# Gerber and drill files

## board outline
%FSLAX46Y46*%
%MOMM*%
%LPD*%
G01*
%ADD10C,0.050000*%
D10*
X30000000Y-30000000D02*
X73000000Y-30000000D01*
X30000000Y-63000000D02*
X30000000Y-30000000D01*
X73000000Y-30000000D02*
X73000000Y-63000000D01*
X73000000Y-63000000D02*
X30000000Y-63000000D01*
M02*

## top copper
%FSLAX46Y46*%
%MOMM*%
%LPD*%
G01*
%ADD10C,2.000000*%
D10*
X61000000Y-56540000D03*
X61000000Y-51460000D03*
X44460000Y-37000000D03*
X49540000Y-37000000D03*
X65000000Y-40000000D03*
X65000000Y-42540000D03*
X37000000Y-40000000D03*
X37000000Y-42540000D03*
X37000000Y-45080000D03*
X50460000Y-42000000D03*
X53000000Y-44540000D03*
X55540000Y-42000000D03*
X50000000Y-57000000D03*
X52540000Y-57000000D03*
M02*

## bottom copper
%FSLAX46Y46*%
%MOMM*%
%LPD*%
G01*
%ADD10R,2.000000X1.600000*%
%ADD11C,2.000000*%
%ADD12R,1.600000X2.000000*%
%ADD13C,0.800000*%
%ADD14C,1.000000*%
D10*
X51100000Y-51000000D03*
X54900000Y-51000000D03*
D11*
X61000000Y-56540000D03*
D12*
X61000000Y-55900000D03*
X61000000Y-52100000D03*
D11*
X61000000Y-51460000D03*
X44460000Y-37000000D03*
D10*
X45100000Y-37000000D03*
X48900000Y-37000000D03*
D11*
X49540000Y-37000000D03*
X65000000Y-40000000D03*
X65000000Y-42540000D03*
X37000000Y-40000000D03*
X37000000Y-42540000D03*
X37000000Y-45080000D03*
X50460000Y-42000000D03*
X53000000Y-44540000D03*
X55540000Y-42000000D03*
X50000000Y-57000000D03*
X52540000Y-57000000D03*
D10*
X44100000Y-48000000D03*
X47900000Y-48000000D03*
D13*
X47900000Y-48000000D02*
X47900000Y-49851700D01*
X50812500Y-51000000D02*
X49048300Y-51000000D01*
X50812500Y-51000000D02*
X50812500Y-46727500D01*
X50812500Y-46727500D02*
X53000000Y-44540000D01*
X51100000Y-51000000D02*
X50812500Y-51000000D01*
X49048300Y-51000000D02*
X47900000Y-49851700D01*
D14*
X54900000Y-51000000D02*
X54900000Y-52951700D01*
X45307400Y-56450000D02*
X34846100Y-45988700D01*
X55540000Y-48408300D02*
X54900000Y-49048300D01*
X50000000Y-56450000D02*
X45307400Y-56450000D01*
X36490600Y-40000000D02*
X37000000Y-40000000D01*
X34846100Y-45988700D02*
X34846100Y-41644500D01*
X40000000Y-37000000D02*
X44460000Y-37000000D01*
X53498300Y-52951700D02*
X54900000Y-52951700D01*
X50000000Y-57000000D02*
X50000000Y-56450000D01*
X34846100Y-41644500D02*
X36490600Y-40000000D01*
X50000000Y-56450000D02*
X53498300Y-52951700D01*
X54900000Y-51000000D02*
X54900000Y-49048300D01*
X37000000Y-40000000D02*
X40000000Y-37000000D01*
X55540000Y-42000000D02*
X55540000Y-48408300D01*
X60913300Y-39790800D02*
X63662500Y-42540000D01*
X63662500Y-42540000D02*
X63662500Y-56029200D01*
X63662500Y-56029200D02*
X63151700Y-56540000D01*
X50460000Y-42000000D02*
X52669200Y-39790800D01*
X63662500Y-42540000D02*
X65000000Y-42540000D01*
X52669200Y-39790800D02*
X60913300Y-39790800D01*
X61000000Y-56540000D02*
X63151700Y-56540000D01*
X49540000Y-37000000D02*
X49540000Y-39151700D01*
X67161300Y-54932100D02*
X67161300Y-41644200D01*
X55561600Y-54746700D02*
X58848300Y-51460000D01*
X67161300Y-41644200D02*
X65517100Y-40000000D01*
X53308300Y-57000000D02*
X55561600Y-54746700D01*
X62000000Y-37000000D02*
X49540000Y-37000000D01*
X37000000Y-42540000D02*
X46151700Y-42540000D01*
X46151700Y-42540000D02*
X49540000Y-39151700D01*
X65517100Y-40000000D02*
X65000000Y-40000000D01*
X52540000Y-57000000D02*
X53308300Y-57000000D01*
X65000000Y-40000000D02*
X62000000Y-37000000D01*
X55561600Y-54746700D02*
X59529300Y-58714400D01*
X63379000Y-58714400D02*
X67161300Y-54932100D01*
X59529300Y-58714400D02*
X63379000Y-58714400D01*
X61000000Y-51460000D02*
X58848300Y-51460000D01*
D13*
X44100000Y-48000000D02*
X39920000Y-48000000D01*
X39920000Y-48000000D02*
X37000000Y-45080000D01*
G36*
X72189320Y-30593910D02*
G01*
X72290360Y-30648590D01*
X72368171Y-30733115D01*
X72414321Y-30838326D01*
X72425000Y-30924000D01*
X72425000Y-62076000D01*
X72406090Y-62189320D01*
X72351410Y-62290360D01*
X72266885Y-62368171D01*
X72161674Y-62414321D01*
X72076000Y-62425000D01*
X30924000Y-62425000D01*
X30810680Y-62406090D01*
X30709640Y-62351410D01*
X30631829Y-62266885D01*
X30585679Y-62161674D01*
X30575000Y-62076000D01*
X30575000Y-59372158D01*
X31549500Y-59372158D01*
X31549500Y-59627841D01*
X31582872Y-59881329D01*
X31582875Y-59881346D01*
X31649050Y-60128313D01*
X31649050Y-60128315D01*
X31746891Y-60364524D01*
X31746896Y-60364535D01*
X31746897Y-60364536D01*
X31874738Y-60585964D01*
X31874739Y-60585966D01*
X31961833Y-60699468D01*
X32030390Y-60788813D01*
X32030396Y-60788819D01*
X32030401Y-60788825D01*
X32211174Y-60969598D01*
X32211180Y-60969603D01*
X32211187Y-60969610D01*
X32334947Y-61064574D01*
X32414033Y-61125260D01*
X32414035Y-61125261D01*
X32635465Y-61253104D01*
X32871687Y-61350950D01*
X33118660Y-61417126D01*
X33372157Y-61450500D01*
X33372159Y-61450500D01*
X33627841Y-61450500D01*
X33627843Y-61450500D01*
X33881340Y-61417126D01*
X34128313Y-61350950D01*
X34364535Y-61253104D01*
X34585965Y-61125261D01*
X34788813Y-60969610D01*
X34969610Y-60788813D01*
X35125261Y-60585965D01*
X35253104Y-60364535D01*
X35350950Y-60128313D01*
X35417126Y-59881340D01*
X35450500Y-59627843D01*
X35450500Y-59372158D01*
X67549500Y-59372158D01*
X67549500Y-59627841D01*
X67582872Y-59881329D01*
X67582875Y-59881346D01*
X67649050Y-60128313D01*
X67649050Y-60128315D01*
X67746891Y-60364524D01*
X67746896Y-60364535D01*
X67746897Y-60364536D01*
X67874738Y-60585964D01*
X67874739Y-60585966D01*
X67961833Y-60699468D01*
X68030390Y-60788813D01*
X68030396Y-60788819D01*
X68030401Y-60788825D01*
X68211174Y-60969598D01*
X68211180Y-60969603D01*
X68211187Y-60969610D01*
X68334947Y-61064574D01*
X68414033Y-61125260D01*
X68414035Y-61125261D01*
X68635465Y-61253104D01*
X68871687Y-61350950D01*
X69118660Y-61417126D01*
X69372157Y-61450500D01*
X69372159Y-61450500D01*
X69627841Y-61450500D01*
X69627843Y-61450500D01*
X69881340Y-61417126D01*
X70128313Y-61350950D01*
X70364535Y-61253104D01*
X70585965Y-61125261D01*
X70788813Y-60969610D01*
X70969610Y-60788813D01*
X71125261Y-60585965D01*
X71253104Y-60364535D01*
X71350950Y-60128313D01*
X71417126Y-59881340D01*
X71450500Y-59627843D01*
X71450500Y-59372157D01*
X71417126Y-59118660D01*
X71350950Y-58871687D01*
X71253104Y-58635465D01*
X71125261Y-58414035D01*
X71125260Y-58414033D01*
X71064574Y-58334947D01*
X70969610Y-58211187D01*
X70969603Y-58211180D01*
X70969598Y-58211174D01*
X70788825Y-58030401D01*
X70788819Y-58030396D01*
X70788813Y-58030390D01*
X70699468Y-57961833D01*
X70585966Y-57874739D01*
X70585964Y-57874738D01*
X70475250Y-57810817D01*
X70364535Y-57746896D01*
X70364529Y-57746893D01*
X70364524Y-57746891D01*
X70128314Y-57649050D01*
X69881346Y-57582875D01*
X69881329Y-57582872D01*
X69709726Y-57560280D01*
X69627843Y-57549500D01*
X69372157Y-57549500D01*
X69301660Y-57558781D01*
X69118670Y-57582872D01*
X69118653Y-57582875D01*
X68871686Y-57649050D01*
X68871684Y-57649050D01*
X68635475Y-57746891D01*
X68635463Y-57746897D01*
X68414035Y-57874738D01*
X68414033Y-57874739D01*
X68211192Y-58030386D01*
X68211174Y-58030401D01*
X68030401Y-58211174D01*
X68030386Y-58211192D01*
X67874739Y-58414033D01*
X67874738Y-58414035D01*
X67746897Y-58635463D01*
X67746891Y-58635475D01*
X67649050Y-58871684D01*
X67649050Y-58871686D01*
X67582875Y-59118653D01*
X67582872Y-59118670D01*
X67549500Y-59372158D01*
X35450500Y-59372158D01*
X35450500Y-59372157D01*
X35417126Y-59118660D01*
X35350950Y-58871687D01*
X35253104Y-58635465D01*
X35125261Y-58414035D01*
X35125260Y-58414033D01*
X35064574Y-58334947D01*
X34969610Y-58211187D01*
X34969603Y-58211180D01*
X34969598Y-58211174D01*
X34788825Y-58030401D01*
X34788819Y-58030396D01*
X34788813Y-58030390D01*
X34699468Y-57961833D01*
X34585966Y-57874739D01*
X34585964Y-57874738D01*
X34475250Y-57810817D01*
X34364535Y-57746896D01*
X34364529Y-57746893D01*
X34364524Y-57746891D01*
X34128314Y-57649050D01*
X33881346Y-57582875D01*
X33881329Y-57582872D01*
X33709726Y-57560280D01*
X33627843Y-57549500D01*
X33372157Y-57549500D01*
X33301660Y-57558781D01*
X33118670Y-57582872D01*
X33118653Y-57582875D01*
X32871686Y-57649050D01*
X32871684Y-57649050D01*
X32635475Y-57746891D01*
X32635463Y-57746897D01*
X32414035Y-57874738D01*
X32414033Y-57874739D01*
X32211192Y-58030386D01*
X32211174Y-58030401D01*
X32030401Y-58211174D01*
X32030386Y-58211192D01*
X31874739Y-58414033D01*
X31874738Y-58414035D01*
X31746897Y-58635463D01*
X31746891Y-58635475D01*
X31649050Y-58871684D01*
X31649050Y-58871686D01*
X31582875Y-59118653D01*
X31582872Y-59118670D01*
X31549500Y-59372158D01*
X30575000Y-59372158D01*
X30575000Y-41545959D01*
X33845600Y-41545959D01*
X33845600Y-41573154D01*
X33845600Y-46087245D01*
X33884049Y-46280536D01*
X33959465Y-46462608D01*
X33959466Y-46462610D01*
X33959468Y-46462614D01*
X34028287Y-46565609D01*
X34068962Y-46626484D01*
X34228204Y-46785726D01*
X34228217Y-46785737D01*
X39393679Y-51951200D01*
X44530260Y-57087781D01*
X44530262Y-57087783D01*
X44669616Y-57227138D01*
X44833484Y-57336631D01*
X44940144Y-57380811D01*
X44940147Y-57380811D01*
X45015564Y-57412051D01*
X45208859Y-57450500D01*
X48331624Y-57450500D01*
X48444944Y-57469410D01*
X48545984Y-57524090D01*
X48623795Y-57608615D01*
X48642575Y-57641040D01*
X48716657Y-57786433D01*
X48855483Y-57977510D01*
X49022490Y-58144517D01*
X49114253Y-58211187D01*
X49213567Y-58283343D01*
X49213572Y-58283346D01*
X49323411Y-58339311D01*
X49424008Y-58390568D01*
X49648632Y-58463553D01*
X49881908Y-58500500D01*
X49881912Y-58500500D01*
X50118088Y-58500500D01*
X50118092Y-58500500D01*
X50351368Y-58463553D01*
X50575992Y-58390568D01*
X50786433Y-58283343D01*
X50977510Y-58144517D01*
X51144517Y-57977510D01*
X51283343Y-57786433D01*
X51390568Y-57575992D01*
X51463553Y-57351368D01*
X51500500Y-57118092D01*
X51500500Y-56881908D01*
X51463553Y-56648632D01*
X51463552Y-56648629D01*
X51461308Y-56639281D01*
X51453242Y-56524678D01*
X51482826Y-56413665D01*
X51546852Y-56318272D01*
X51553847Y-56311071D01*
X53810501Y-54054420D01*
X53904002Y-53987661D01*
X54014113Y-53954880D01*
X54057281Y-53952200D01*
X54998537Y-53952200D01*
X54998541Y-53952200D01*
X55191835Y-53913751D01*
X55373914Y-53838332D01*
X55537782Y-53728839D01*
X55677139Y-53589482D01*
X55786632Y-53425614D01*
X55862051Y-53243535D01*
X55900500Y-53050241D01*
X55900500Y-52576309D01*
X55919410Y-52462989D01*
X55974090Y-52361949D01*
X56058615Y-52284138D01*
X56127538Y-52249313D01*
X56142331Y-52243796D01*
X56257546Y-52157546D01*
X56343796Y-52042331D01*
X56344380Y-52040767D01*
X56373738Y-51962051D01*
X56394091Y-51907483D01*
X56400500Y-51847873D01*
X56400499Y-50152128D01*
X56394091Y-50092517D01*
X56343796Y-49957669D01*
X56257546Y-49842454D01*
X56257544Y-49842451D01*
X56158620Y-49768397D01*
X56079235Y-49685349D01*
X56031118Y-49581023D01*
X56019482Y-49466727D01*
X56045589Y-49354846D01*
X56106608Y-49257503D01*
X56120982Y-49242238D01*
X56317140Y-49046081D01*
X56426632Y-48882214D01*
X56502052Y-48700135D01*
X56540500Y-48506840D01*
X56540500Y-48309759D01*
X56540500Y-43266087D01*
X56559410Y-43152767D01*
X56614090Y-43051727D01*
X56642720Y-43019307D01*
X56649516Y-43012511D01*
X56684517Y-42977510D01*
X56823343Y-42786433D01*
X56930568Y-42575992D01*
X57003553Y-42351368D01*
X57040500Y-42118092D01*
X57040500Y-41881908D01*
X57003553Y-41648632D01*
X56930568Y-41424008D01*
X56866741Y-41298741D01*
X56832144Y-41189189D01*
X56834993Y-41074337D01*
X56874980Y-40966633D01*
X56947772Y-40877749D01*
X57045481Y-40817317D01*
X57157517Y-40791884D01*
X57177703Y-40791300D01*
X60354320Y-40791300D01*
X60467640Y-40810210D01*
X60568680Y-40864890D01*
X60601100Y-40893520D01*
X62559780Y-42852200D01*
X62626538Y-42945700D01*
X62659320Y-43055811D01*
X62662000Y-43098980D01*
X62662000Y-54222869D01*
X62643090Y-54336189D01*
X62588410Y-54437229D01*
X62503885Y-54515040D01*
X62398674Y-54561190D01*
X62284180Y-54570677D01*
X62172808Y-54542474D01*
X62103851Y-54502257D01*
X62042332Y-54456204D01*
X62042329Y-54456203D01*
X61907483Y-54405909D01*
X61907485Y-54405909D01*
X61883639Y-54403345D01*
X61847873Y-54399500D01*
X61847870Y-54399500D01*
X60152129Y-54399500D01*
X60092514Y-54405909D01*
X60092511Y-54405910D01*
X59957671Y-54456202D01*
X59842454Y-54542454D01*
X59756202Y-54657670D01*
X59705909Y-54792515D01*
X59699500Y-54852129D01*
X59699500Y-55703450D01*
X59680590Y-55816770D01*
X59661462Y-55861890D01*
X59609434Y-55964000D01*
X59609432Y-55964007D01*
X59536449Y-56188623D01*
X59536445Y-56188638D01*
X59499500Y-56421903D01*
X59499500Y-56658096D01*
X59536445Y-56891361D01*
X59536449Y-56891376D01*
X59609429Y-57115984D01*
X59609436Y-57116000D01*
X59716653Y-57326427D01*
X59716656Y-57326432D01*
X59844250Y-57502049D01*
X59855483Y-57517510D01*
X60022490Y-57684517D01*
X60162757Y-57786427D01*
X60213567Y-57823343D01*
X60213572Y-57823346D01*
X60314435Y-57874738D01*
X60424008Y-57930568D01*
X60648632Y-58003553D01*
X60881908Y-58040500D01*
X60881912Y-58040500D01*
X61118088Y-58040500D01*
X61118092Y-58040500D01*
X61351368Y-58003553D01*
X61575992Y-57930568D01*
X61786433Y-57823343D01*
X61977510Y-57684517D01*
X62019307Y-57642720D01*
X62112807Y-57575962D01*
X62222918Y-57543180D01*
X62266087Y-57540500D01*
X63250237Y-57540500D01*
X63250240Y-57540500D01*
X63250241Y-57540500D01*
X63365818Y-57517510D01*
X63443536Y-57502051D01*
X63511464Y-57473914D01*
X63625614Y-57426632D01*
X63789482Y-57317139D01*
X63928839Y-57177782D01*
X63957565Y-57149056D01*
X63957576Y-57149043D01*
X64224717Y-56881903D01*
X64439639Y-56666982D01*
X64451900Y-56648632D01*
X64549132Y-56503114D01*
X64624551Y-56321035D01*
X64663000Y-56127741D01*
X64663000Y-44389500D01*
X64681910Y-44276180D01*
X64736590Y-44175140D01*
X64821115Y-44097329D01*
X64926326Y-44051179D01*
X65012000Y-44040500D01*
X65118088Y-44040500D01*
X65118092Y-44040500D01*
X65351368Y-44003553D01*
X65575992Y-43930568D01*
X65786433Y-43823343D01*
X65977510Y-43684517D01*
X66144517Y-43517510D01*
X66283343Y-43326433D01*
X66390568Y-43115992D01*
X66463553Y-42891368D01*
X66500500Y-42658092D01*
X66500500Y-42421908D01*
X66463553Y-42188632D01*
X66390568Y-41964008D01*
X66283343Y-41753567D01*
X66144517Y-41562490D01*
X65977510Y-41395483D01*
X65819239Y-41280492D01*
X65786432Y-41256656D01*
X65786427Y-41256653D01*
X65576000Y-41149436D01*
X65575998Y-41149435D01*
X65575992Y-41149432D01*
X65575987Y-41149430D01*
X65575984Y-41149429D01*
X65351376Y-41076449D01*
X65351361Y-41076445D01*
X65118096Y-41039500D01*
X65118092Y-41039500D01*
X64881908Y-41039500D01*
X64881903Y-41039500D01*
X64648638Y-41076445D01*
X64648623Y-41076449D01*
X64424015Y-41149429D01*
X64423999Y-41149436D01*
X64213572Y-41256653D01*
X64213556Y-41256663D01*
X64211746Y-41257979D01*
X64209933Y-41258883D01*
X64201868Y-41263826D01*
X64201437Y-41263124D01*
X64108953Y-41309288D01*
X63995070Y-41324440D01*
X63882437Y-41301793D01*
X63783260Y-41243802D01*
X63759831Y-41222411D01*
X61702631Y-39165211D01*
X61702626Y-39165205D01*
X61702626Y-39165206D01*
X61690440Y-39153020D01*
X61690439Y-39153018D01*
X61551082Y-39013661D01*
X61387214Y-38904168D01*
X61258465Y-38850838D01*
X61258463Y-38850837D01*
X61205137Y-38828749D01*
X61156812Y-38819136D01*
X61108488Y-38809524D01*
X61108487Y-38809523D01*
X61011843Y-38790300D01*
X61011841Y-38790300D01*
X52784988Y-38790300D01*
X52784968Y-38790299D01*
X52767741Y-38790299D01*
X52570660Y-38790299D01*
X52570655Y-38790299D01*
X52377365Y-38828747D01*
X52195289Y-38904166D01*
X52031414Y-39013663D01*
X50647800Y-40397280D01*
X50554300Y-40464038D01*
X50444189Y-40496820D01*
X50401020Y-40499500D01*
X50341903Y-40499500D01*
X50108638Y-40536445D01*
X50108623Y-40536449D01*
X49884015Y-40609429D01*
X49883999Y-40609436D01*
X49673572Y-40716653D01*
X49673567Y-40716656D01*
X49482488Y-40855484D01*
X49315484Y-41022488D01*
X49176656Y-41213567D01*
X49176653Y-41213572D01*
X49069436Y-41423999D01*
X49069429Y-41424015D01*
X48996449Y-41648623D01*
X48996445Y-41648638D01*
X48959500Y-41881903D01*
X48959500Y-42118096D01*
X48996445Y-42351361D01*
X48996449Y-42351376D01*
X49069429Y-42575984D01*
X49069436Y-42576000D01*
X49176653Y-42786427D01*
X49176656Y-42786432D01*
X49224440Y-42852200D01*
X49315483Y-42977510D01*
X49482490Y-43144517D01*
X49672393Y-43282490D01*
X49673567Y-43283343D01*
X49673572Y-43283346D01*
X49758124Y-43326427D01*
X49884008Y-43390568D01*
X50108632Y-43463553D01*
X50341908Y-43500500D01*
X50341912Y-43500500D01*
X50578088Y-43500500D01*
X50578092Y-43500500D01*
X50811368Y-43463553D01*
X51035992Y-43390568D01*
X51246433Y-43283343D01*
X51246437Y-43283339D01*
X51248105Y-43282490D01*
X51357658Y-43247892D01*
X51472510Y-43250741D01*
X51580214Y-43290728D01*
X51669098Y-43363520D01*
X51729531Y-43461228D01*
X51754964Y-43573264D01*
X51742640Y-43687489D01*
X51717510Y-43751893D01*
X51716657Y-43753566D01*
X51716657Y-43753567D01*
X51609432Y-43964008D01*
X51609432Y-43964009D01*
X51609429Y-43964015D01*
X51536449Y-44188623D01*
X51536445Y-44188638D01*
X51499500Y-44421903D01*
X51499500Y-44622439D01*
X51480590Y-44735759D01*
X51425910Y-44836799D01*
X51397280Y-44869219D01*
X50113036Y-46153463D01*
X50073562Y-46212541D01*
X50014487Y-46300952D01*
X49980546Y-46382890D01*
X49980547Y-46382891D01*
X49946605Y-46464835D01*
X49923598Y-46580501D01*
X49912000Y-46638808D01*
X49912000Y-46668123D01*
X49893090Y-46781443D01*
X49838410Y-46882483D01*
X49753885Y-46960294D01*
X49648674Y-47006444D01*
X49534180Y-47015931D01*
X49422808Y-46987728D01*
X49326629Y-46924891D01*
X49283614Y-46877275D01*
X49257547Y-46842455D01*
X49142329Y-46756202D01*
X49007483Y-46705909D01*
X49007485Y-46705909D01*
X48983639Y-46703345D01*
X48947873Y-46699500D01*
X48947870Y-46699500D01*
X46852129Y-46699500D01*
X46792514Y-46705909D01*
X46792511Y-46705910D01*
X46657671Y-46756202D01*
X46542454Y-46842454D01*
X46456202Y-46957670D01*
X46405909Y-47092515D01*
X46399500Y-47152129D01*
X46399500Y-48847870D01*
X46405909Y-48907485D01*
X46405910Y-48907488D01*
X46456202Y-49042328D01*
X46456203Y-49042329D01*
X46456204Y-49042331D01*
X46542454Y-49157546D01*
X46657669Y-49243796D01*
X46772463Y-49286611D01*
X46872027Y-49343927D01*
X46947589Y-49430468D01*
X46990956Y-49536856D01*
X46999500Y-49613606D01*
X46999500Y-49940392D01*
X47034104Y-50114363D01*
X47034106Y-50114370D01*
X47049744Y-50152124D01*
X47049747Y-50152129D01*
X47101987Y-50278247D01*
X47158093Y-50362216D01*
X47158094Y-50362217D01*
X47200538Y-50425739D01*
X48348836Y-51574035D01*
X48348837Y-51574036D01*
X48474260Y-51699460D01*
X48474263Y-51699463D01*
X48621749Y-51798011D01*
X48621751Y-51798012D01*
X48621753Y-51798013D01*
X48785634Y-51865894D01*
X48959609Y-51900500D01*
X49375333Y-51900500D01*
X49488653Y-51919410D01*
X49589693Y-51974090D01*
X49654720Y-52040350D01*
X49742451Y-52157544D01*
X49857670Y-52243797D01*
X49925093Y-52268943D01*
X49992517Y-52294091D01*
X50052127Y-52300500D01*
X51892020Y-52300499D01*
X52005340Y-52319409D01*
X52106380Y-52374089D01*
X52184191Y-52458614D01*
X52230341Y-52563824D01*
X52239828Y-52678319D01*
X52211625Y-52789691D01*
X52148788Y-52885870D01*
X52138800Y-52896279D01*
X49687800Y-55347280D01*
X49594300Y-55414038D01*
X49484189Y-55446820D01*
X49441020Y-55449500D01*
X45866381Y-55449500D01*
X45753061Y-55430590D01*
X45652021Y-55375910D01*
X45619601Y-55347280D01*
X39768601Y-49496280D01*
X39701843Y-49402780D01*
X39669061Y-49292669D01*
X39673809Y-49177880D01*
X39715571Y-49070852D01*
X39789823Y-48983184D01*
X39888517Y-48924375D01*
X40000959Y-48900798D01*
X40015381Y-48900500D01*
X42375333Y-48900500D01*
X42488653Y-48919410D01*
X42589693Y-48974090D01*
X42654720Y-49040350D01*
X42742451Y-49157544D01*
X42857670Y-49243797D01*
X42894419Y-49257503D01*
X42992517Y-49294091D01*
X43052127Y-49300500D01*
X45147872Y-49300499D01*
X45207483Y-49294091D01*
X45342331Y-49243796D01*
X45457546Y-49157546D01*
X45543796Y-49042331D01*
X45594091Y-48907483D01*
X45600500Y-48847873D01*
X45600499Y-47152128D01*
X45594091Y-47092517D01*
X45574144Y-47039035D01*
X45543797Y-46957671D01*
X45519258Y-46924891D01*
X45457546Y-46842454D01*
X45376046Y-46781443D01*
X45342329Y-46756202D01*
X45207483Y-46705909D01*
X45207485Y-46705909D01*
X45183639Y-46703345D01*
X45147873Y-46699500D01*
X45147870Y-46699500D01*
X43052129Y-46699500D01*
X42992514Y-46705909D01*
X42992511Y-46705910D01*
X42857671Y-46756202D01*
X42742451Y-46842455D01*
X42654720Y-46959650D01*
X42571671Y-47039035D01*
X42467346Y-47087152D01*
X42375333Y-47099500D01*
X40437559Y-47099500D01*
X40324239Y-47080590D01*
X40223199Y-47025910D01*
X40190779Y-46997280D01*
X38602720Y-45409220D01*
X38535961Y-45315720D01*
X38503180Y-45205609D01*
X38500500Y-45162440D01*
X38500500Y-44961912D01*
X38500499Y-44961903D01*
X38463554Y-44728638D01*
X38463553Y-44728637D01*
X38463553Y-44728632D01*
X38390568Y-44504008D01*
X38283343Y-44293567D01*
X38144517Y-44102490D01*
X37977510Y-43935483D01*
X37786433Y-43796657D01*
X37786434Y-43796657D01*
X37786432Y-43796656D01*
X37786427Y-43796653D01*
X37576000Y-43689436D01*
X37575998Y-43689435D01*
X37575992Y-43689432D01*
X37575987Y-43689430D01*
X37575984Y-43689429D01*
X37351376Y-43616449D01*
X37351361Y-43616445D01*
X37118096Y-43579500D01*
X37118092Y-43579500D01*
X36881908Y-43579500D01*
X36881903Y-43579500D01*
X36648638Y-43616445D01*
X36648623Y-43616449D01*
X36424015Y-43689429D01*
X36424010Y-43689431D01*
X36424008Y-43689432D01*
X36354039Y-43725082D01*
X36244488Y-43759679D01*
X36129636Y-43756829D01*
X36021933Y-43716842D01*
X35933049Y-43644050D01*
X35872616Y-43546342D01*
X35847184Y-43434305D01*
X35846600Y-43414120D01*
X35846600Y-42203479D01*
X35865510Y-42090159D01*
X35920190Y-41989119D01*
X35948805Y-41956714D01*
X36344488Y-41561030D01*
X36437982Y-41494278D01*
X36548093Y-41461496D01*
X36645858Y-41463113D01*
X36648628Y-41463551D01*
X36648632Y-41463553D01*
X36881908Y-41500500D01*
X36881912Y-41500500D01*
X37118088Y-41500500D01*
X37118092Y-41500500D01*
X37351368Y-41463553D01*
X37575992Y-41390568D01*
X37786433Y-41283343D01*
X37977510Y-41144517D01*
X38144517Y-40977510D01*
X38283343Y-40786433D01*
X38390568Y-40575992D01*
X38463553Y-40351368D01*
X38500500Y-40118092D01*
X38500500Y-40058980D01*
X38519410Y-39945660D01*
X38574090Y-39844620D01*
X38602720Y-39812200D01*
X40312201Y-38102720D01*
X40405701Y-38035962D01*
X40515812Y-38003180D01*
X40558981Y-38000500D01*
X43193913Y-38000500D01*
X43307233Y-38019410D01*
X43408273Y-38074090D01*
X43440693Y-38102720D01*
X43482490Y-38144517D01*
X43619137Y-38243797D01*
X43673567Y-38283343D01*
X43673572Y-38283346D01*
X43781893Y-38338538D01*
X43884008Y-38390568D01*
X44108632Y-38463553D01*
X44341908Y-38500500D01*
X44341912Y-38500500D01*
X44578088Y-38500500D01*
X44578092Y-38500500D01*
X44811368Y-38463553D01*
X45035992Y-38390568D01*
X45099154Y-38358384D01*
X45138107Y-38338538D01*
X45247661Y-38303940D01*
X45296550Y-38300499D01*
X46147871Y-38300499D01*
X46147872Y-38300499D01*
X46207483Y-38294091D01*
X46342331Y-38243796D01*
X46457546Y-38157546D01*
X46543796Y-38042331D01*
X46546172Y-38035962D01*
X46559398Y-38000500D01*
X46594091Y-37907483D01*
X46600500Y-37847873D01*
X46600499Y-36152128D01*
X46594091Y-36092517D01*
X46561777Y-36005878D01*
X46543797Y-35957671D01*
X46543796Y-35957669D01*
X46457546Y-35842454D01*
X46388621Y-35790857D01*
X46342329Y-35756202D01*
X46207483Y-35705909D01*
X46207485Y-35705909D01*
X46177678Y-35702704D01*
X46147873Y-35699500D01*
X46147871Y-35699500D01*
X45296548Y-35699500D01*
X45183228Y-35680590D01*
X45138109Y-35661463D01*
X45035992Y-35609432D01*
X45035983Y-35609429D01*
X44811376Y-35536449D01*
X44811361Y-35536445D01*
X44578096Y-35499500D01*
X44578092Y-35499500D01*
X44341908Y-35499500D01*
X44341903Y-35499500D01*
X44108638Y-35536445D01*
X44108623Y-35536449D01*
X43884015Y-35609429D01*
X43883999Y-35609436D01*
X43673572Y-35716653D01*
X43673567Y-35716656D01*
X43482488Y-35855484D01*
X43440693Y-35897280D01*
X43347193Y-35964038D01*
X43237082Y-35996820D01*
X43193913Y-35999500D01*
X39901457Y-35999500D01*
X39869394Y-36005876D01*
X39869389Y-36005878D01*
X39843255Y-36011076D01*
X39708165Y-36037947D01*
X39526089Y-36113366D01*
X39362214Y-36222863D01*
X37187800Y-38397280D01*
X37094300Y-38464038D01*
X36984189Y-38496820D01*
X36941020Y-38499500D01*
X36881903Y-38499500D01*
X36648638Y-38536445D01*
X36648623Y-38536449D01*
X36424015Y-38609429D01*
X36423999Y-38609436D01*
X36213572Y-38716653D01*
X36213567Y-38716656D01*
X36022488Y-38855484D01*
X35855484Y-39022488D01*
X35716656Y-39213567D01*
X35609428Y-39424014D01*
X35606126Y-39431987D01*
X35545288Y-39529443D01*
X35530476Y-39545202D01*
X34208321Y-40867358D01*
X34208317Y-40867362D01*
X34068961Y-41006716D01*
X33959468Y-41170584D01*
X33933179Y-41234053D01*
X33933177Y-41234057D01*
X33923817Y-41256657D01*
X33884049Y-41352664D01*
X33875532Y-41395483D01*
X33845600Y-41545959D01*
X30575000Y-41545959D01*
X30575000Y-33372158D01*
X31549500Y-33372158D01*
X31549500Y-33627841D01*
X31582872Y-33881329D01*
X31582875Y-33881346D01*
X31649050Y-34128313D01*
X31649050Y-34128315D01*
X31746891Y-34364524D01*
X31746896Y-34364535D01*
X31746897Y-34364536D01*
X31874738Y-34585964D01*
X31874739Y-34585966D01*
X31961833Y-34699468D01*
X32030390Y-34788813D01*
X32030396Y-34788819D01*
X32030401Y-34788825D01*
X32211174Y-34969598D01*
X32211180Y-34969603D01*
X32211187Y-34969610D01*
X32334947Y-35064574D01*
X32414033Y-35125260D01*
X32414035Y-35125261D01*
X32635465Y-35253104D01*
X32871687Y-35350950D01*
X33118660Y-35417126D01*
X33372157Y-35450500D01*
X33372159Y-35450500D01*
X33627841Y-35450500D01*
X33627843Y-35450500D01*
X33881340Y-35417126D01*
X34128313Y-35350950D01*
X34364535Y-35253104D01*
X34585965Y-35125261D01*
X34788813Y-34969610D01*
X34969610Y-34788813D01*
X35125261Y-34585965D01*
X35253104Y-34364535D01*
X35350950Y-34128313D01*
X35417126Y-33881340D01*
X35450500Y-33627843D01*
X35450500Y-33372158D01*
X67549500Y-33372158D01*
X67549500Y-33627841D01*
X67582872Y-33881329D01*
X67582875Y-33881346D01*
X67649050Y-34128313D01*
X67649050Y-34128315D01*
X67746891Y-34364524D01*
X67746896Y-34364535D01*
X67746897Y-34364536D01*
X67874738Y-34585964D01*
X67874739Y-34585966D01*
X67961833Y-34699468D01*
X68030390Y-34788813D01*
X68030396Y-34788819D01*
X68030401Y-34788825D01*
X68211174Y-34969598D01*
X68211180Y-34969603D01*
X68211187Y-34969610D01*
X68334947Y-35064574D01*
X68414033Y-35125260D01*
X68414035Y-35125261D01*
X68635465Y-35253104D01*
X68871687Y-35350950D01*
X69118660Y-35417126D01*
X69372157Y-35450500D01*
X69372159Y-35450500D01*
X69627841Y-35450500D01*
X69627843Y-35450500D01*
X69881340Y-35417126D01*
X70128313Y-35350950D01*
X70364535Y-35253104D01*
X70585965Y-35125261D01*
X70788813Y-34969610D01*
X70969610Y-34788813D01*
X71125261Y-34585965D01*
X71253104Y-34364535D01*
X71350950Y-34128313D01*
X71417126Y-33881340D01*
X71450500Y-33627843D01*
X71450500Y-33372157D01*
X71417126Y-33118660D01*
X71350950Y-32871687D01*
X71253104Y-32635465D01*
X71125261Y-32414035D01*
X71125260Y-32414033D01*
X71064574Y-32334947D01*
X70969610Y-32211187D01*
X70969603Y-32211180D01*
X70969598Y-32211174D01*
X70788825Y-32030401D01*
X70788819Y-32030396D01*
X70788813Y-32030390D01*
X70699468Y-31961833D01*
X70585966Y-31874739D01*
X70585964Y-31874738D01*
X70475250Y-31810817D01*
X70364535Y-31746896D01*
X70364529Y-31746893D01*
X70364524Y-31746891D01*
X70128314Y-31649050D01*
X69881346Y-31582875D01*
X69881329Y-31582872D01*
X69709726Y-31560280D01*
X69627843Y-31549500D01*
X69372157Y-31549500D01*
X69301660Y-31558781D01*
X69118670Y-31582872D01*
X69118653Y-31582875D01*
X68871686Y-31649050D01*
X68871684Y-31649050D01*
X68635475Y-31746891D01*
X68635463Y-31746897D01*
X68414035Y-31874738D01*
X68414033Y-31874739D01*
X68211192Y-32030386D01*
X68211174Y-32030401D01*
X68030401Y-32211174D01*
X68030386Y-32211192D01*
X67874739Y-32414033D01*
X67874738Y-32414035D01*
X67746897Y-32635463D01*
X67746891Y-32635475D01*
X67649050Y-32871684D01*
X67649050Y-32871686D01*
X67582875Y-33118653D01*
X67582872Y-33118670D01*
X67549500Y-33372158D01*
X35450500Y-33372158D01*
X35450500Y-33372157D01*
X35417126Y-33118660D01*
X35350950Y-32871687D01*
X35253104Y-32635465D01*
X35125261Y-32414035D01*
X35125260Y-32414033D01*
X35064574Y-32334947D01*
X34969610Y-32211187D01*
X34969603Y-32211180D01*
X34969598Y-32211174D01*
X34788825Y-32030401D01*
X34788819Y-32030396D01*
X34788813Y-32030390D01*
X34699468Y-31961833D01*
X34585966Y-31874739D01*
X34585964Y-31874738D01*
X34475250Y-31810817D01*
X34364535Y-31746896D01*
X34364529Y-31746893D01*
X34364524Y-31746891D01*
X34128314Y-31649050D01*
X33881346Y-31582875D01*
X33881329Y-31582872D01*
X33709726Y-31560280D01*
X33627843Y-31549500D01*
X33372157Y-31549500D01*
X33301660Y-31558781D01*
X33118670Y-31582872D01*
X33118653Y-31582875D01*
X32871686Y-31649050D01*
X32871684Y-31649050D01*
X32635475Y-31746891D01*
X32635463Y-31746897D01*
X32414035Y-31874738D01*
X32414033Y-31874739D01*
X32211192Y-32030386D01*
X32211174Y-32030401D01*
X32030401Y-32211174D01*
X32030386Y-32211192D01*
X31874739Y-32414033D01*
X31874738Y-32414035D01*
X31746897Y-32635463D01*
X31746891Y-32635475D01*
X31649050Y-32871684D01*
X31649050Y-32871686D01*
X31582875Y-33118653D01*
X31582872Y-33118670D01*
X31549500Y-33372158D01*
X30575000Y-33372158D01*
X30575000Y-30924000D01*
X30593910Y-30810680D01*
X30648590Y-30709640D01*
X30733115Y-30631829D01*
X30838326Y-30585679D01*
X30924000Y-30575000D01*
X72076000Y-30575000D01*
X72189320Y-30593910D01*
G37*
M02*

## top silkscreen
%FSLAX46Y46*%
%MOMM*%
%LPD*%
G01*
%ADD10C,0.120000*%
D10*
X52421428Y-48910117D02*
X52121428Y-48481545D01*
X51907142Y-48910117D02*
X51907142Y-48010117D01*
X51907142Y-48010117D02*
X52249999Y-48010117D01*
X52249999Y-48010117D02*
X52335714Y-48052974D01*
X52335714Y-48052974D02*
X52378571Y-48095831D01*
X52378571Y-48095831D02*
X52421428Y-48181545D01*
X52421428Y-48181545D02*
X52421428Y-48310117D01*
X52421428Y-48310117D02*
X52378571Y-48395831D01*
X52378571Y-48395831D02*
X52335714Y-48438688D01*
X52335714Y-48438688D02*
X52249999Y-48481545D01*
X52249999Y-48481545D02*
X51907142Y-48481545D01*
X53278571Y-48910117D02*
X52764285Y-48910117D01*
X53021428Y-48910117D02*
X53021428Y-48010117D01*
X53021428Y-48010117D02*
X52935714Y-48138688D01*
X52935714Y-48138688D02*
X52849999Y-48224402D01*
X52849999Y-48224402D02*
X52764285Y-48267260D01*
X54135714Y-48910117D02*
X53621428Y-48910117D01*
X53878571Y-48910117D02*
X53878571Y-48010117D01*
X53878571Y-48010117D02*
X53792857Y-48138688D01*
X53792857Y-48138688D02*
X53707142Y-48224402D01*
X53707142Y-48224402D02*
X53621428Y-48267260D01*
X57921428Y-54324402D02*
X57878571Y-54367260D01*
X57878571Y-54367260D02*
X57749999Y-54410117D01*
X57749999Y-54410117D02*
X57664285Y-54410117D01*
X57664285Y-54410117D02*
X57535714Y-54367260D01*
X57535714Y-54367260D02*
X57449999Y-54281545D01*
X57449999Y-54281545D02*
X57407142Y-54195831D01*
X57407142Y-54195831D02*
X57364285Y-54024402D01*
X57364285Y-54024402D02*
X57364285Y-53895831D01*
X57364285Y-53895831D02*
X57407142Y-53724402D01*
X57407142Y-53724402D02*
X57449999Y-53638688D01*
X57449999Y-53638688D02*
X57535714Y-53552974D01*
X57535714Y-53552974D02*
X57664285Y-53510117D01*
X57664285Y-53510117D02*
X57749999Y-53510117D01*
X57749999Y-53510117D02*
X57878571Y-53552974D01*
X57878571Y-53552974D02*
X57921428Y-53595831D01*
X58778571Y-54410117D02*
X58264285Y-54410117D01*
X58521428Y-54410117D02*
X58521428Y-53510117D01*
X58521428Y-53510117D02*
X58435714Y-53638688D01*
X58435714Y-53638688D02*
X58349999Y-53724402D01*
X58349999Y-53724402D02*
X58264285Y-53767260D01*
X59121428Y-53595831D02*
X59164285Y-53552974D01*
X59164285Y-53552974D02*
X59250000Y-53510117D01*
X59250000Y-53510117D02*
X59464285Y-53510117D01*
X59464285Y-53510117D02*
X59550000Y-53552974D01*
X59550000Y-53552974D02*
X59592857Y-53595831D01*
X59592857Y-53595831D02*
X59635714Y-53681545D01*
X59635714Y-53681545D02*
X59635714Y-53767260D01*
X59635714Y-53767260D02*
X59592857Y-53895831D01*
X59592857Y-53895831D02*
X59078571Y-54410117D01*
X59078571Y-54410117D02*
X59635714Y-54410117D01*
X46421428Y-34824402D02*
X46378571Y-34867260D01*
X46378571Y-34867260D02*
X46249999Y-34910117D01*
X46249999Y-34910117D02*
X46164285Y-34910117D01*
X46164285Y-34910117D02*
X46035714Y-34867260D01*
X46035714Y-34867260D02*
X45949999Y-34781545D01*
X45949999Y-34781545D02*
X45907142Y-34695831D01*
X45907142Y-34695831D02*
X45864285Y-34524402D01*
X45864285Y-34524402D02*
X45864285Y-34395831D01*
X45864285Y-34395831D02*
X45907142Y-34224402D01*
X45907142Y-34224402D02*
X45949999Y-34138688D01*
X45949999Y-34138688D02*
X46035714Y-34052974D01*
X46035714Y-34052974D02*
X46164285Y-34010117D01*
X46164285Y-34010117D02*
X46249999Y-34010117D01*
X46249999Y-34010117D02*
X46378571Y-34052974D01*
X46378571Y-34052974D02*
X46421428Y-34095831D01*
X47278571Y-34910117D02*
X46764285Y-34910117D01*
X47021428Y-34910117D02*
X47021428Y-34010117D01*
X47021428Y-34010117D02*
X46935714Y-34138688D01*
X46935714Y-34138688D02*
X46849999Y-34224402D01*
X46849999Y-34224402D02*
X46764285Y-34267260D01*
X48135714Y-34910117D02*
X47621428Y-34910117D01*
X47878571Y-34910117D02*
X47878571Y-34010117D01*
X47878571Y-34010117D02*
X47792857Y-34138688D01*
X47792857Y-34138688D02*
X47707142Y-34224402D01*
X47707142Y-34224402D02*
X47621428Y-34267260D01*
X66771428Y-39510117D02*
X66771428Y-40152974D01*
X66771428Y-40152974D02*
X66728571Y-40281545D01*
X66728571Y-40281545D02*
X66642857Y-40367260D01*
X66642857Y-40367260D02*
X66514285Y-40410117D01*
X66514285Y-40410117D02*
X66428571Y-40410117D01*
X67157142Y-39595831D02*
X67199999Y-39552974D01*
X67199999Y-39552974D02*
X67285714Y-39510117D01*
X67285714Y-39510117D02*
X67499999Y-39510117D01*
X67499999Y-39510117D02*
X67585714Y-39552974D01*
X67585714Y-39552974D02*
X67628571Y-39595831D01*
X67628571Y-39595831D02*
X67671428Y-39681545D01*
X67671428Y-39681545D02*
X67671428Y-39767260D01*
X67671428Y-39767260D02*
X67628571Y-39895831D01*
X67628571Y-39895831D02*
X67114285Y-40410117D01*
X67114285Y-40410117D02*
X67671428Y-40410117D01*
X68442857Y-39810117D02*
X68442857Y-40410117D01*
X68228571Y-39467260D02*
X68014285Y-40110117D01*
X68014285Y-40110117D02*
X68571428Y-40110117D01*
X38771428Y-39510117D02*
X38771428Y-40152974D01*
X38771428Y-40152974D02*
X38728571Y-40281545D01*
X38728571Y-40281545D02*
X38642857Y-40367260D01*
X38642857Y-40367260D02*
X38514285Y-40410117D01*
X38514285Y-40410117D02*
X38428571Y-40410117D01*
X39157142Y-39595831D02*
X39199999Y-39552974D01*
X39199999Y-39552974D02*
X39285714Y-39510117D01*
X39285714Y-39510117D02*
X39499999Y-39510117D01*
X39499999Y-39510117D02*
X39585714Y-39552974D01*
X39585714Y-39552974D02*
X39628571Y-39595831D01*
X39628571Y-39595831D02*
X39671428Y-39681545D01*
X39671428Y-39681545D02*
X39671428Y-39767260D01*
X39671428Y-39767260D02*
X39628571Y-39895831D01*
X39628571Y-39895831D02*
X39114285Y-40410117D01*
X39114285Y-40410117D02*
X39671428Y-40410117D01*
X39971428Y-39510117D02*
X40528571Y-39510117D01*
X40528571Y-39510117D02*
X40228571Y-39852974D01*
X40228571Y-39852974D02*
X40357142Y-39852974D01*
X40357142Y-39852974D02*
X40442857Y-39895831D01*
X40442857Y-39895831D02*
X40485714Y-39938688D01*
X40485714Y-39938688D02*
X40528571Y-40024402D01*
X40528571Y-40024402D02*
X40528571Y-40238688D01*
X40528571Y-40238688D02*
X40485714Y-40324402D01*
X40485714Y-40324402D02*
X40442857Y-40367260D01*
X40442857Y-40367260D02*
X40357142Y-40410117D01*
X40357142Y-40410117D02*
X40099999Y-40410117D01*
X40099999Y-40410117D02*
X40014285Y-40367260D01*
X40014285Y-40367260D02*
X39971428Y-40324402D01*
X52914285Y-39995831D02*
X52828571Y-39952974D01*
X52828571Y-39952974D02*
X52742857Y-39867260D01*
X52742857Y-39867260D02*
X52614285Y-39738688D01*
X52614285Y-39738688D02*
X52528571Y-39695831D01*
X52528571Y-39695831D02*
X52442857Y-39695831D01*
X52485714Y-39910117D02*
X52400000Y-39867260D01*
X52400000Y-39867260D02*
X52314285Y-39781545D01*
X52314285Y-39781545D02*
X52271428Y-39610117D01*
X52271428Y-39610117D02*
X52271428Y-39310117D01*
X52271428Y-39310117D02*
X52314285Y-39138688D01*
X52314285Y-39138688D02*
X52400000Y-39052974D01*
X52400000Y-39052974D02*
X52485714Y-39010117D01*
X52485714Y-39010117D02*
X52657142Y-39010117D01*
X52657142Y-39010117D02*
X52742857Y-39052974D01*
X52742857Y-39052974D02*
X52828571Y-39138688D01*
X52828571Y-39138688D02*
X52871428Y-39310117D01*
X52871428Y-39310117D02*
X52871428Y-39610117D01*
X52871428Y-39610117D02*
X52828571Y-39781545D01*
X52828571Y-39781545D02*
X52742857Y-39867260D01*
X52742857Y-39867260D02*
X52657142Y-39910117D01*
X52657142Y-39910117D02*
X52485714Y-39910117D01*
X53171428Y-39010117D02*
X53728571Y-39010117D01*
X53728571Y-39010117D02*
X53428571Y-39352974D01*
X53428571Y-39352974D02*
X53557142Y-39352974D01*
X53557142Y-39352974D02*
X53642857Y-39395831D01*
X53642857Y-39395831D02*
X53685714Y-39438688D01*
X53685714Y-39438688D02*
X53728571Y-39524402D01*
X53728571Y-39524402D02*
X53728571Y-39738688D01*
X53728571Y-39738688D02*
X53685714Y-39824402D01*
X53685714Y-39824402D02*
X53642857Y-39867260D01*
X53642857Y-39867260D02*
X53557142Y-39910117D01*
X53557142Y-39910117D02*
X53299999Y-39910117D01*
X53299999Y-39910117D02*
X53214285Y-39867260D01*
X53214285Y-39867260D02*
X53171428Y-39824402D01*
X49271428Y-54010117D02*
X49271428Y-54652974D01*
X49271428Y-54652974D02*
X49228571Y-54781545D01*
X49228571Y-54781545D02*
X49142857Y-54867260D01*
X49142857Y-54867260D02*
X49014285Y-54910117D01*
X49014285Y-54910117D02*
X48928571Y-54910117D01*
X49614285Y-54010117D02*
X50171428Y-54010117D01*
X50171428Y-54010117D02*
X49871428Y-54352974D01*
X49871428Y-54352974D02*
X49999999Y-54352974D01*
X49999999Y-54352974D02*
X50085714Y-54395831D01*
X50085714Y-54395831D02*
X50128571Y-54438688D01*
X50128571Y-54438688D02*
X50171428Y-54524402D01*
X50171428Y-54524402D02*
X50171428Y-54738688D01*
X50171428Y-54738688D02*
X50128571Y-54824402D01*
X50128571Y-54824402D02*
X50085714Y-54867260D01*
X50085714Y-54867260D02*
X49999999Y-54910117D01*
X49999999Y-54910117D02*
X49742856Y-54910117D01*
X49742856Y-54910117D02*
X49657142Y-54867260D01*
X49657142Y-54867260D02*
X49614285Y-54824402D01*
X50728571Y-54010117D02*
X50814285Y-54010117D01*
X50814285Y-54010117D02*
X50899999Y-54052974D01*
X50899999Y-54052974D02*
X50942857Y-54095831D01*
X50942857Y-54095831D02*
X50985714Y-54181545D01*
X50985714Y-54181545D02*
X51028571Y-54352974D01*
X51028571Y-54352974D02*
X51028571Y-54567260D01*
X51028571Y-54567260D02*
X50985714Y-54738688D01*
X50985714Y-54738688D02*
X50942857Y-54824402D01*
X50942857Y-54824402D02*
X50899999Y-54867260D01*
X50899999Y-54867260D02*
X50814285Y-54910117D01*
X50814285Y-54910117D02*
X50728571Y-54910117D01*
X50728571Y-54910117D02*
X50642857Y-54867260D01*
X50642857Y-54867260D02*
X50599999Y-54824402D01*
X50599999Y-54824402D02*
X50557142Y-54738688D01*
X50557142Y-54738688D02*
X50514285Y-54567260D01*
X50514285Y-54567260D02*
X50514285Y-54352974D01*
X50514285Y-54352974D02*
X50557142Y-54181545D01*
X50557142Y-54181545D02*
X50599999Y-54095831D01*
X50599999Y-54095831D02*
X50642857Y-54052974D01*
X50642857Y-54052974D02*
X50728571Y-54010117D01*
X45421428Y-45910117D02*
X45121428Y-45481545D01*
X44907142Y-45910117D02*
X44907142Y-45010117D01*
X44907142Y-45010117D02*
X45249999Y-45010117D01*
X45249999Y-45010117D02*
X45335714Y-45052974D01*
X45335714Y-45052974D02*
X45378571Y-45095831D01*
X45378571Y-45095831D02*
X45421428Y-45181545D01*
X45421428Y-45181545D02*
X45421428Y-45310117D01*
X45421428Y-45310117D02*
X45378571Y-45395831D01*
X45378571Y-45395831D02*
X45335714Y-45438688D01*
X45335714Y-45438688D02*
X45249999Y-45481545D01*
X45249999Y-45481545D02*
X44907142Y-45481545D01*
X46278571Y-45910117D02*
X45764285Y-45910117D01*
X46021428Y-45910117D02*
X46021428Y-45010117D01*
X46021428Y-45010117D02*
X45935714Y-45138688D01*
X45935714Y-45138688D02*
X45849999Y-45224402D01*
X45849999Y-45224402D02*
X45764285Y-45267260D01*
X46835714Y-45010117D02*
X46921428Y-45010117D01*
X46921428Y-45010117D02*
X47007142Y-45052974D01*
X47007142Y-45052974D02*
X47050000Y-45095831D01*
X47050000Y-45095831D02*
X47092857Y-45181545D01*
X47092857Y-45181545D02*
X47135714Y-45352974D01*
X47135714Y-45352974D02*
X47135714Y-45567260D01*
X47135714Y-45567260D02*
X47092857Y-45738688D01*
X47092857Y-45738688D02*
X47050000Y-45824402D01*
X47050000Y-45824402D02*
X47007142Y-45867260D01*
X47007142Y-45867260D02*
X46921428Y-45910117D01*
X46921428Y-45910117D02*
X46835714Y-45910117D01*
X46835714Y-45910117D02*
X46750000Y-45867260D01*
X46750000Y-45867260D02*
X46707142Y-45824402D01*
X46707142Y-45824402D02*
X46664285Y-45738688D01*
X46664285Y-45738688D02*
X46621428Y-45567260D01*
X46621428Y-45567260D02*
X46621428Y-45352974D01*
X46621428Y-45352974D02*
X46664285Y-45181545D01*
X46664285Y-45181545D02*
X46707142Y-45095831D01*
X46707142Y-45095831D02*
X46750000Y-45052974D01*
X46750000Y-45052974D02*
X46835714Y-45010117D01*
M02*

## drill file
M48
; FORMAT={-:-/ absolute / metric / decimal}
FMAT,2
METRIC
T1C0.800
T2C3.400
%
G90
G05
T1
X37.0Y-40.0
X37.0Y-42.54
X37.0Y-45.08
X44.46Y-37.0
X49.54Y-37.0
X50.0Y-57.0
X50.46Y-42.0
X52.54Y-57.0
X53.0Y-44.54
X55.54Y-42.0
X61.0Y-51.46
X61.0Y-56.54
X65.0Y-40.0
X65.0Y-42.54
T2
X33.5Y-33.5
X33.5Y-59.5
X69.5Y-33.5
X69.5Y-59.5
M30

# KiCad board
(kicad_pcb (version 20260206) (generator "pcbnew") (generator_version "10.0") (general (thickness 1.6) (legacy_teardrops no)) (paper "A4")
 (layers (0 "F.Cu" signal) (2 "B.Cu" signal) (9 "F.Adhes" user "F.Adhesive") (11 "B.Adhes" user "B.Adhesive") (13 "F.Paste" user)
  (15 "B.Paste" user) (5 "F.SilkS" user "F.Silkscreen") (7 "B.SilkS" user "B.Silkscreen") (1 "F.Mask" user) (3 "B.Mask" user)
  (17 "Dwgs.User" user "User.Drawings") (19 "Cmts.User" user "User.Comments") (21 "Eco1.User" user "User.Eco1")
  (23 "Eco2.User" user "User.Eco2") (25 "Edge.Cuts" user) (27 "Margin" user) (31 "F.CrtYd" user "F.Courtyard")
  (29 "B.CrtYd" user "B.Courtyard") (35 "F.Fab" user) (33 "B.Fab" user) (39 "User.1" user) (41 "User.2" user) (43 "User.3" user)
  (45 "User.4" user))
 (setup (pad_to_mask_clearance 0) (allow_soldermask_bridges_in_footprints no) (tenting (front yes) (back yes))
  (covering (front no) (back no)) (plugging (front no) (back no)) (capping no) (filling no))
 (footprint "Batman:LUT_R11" (layer "F.Cu") (at 53 51)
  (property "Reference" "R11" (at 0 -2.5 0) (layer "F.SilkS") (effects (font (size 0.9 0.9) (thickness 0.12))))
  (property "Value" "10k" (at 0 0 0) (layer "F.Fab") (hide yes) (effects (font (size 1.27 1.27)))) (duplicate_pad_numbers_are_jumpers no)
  (pad "1" smd rect (at -1.9 0) (size 2 1.6) (layers "B.Cu") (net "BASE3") (thermal_bridge_angle 45))
  (pad "2" smd rect (at 1.9 0) (size 2 1.6) (layers "B.Cu") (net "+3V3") (thermal_bridge_angle 45)))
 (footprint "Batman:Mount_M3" (layer "F.Cu") (at 69.5 33.5)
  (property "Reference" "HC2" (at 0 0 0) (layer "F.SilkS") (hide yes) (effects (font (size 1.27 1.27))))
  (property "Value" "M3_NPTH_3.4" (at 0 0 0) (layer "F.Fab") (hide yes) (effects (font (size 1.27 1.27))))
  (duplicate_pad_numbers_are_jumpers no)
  (pad "" np_thru_hole circle (at 0 0) (size 3.4 3.4) (drill 3.4) (layers "*.Cu")))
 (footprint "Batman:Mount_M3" (layer "F.Cu") (at 33.5 59.5)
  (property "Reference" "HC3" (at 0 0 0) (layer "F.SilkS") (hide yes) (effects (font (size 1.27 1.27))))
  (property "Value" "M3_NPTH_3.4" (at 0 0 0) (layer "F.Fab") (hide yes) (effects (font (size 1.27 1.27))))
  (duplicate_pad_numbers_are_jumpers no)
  (pad "" np_thru_hole circle (at 0 0) (size 3.4 3.4) (drill 3.4) (layers "*.Cu")))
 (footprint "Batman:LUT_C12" (layer "F.Cu") (at 61 54 90)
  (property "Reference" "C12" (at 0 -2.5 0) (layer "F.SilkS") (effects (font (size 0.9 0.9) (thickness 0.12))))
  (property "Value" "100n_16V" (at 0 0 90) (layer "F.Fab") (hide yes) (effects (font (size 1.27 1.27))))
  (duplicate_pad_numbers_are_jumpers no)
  (pad "1" thru_hole circle (at -2.54 0 90) (size 2 2) (drill 0.8) (layers "*.Cu") (remove_unused_layers no) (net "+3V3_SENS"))
  (pad "1" smd rect (at -1.9 0 90) (size 2 1.6) (layers "B.Cu") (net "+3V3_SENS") (thermal_bridge_angle 45))
  (pad "2" smd rect (at 1.9 0 90) (size 2 1.6) (layers "B.Cu") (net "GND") (thermal_bridge_angle 45))
  (pad "2" thru_hole circle (at 2.54 0 90) (size 2 2) (drill 0.8) (layers "*.Cu") (remove_unused_layers no) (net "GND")))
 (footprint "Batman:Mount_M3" (layer "F.Cu") (at 33.5 33.5)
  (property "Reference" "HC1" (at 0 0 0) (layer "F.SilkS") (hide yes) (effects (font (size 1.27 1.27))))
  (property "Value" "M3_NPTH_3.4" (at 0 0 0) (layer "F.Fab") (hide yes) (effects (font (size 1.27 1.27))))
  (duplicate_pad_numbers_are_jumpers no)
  (pad "" np_thru_hole circle (at 0 0) (size 3.4 3.4) (drill 3.4) (layers "*.Cu")))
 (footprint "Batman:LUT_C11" (layer "F.Cu") (at 47 37)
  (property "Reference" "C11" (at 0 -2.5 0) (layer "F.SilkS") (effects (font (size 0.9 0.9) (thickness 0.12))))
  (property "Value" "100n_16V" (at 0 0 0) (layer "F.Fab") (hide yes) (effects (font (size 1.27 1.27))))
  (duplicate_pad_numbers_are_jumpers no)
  (pad "1" thru_hole circle (at -2.54 0) (size 2 2) (drill 0.8) (layers "*.Cu") (remove_unused_layers no) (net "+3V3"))
  (pad "1" smd rect (at -1.9 0) (size 2 1.6) (layers "B.Cu") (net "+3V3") (thermal_bridge_angle 45))
  (pad "2" smd rect (at 1.9 0) (size 2 1.6) (layers "B.Cu") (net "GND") (thermal_bridge_angle 45))
  (pad "2" thru_hole circle (at 2.54 0) (size 2 2) (drill 0.8) (layers "*.Cu") (remove_unused_layers no) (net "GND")))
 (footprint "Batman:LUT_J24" (layer "F.Cu") (at 65 40 -90)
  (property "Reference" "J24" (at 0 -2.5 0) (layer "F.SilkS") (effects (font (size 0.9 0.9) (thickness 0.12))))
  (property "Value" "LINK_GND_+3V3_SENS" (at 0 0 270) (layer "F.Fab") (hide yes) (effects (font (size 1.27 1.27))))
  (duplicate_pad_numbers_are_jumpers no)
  (pad "1" thru_hole circle (at 0 0 270) (size 2 2) (drill 0.8) (layers "*.Cu") (remove_unused_layers no) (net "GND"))
  (pad "2" thru_hole circle (at 2.54 0 270) (size 2 2) (drill 0.8) (layers "*.Cu") (remove_unused_layers no) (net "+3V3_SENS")))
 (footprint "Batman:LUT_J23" (layer "F.Cu") (at 37 40 -90)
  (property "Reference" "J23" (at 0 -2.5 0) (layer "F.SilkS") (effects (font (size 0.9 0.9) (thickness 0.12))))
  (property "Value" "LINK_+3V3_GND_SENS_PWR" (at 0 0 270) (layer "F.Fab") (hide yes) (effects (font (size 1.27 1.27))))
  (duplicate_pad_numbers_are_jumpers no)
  (pad "1" thru_hole circle (at 0 0 270) (size 2 2) (drill 0.8) (layers "*.Cu") (remove_unused_layers no) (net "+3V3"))
  (pad "2" thru_hole circle (at 2.54 0 270) (size 2 2) (drill 0.8) (layers "*.Cu") (remove_unused_layers no) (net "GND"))
  (pad "3" thru_hole circle (at 5.08 0 270) (size 2 2) (drill 0.8) (layers "*.Cu") (remove_unused_layers no) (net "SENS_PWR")))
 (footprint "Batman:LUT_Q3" (layer "F.Cu") (at 53 42)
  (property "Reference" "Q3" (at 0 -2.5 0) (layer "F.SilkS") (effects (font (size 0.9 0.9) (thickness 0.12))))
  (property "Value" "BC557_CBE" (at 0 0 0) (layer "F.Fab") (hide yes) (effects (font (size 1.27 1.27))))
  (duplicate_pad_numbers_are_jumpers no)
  (pad "1" thru_hole circle (at -2.54 0) (size 2 2) (drill 0.8) (layers "*.Cu") (remove_unused_layers no) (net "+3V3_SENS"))
  (pad "2" thru_hole circle (at 0 2.54) (size 2 2) (drill 0.8) (layers "*.Cu") (remove_unused_layers no) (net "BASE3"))
  (pad "3" thru_hole circle (at 2.54 0) (size 2 2) (drill 0.8) (layers "*.Cu") (remove_unused_layers no) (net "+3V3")))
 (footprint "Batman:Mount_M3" (layer "F.Cu") (at 69.5 59.5)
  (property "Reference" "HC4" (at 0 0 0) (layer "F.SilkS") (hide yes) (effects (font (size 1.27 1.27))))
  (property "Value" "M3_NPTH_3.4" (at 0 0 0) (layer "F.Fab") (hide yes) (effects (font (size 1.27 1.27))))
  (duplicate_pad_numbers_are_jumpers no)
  (pad "" np_thru_hole circle (at 0 0) (size 3.4 3.4) (drill 3.4) (layers "*.Cu")))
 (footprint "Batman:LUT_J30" (layer "F.Cu") (at 50 57)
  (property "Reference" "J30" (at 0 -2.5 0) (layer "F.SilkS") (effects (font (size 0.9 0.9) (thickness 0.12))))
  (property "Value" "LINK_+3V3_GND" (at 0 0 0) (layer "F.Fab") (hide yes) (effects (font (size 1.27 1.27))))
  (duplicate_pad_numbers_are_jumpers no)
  (pad "1" thru_hole circle (at 0 0) (size 2 2) (drill 0.8) (layers "*.Cu") (remove_unused_layers no) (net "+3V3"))
  (pad "2" thru_hole circle (at 2.54 0) (size 2 2) (drill 0.8) (layers "*.Cu") (remove_unused_layers no) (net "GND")))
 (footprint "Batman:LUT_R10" (layer "F.Cu") (at 46 48)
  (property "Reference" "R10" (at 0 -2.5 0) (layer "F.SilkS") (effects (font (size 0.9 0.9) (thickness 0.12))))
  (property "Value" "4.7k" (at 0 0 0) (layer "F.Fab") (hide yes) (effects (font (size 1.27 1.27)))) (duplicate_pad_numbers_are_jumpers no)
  (pad "1" smd rect (at -1.9 0) (size 2 1.6) (layers "B.Cu") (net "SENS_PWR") (thermal_bridge_angle 45))
  (pad "2" smd rect (at 1.9 0) (size 2 1.6) (layers "B.Cu") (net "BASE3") (thermal_bridge_angle 45)))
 (gr_line (start 30 30) (end 73 30) (stroke (width 0.05) (type default)) (layer "Edge.Cuts"))
 (gr_line (start 30 63) (end 30 30) (stroke (width 0.05) (type default)) (layer "Edge.Cuts"))
 (gr_line (start 73 30) (end 73 63) (stroke (width 0.05) (type default)) (layer "Edge.Cuts"))
 (gr_line (start 73 63) (end 30 63) (stroke (width 0.05) (type default)) (layer "Edge.Cuts"))
 (segment (start 47.9 48) (end 47.9 49.8517) (width 0.8) (layer "B.Cu") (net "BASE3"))
 (segment (start 50.8125 51) (end 49.0483 51) (width 0.8) (layer "B.Cu") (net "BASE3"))
 (segment (start 50.8125 51) (end 50.8125 46.7275) (width 0.8) (layer "B.Cu") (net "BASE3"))
 (segment (start 50.8125 46.7275) (end 53 44.54) (width 0.8) (layer "B.Cu") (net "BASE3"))
 (segment (start 51.1 51) (end 50.8125 51) (width 0.8) (layer "B.Cu") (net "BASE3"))
 (segment (start 49.0483 51) (end 47.9 49.8517) (width 0.8) (layer "B.Cu") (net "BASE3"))
 (segment (start 54.9 51) (end 54.9 52.9517) (width 1) (layer "B.Cu") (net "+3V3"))
 (segment (start 45.3074 56.45) (end 34.8461 45.9887) (width 1) (layer "B.Cu") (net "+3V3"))
 (segment (start 55.54 48.4083) (end 54.9 49.0483) (width 1) (layer "B.Cu") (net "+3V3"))
 (segment (start 50 56.45) (end 45.3074 56.45) (width 1) (layer "B.Cu") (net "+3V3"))
 (segment (start 36.4906 40) (end 37 40) (width 1) (layer "B.Cu") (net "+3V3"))
 (segment (start 34.8461 45.9887) (end 34.8461 41.6445) (width 1) (layer "B.Cu") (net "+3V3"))
 (segment (start 40 37) (end 44.46 37) (width 1) (layer "B.Cu") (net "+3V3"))
 (segment (start 53.4983 52.9517) (end 54.9 52.9517) (width 1) (layer "B.Cu") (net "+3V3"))
 (segment (start 50 57) (end 50 56.45) (width 1) (layer "B.Cu") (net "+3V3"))
 (segment (start 34.8461 41.6445) (end 36.4906 40) (width 1) (layer "B.Cu") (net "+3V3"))
 (segment (start 50 56.45) (end 53.4983 52.9517) (width 1) (layer "B.Cu") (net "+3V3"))
 (segment (start 54.9 51) (end 54.9 49.0483) (width 1) (layer "B.Cu") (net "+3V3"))
 (segment (start 37 40) (end 40 37) (width 1) (layer "B.Cu") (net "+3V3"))
 (segment (start 55.54 42) (end 55.54 48.4083) (width 1) (layer "B.Cu") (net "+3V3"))
 (segment (start 60.9133 39.7908) (end 63.6625 42.54) (width 1) (layer "B.Cu") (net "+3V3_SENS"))
 (segment (start 63.6625 42.54) (end 63.6625 56.0292) (width 1) (layer "B.Cu") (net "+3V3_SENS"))
 (segment (start 63.6625 56.0292) (end 63.1517 56.54) (width 1) (layer "B.Cu") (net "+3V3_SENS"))
 (segment (start 50.46 42) (end 52.6692 39.7908) (width 1) (layer "B.Cu") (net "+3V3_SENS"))
 (segment (start 63.6625 42.54) (end 65 42.54) (width 1) (layer "B.Cu") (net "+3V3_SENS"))
 (segment (start 52.6692 39.7908) (end 60.9133 39.7908) (width 1) (layer "B.Cu") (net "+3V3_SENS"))
 (segment (start 61 56.54) (end 63.1517 56.54) (width 1) (layer "B.Cu") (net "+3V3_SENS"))
 (segment (start 49.54 37) (end 49.54 39.1517) (width 1) (layer "B.Cu") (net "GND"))
 (segment (start 67.1613 54.9321) (end 67.1613 41.6442) (width 1) (layer "B.Cu") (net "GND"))
 (segment (start 55.5616 54.7467) (end 58.8483 51.46) (width 1) (layer "B.Cu") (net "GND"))
 (segment (start 67.1613 41.6442) (end 65.5171 40) (width 1) (layer "B.Cu") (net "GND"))
 (segment (start 53.3083 57) (end 55.5616 54.7467) (width 1) (layer "B.Cu") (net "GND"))
 (segment (start 62 37) (end 49.54 37) (width 1) (layer "B.Cu") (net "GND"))
 (segment (start 37 42.54) (end 46.1517 42.54) (width 1) (layer "B.Cu") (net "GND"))
 (segment (start 46.1517 42.54) (end 49.54 39.1517) (width 1) (layer "B.Cu") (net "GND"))
 (segment (start 65.5171 40) (end 65 40) (width 1) (layer "B.Cu") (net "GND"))
 (segment (start 52.54 57) (end 53.3083 57) (width 1) (layer "B.Cu") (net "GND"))
 (segment (start 65 40) (end 62 37) (width 1) (layer "B.Cu") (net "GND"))
 (segment (start 55.5616 54.7467) (end 59.5293 58.7144) (width 1) (layer "B.Cu") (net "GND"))
 (segment (start 63.379 58.7144) (end 67.1613 54.9321) (width 1) (layer "B.Cu") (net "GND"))
 (segment (start 59.5293 58.7144) (end 63.379 58.7144) (width 1) (layer "B.Cu") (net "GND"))
 (segment (start 61 51.46) (end 58.8483 51.46) (width 1) (layer "B.Cu") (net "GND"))
 (segment (start 44.1 48) (end 39.92 48) (width 0.8) (layer "B.Cu") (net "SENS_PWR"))
 (segment (start 39.92 48) (end 37 45.08) (width 0.8) (layer "B.Cu") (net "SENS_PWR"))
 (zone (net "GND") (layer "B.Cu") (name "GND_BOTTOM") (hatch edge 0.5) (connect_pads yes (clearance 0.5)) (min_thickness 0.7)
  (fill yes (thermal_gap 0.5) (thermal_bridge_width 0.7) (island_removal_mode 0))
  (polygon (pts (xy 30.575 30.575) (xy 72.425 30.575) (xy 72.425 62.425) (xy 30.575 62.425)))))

